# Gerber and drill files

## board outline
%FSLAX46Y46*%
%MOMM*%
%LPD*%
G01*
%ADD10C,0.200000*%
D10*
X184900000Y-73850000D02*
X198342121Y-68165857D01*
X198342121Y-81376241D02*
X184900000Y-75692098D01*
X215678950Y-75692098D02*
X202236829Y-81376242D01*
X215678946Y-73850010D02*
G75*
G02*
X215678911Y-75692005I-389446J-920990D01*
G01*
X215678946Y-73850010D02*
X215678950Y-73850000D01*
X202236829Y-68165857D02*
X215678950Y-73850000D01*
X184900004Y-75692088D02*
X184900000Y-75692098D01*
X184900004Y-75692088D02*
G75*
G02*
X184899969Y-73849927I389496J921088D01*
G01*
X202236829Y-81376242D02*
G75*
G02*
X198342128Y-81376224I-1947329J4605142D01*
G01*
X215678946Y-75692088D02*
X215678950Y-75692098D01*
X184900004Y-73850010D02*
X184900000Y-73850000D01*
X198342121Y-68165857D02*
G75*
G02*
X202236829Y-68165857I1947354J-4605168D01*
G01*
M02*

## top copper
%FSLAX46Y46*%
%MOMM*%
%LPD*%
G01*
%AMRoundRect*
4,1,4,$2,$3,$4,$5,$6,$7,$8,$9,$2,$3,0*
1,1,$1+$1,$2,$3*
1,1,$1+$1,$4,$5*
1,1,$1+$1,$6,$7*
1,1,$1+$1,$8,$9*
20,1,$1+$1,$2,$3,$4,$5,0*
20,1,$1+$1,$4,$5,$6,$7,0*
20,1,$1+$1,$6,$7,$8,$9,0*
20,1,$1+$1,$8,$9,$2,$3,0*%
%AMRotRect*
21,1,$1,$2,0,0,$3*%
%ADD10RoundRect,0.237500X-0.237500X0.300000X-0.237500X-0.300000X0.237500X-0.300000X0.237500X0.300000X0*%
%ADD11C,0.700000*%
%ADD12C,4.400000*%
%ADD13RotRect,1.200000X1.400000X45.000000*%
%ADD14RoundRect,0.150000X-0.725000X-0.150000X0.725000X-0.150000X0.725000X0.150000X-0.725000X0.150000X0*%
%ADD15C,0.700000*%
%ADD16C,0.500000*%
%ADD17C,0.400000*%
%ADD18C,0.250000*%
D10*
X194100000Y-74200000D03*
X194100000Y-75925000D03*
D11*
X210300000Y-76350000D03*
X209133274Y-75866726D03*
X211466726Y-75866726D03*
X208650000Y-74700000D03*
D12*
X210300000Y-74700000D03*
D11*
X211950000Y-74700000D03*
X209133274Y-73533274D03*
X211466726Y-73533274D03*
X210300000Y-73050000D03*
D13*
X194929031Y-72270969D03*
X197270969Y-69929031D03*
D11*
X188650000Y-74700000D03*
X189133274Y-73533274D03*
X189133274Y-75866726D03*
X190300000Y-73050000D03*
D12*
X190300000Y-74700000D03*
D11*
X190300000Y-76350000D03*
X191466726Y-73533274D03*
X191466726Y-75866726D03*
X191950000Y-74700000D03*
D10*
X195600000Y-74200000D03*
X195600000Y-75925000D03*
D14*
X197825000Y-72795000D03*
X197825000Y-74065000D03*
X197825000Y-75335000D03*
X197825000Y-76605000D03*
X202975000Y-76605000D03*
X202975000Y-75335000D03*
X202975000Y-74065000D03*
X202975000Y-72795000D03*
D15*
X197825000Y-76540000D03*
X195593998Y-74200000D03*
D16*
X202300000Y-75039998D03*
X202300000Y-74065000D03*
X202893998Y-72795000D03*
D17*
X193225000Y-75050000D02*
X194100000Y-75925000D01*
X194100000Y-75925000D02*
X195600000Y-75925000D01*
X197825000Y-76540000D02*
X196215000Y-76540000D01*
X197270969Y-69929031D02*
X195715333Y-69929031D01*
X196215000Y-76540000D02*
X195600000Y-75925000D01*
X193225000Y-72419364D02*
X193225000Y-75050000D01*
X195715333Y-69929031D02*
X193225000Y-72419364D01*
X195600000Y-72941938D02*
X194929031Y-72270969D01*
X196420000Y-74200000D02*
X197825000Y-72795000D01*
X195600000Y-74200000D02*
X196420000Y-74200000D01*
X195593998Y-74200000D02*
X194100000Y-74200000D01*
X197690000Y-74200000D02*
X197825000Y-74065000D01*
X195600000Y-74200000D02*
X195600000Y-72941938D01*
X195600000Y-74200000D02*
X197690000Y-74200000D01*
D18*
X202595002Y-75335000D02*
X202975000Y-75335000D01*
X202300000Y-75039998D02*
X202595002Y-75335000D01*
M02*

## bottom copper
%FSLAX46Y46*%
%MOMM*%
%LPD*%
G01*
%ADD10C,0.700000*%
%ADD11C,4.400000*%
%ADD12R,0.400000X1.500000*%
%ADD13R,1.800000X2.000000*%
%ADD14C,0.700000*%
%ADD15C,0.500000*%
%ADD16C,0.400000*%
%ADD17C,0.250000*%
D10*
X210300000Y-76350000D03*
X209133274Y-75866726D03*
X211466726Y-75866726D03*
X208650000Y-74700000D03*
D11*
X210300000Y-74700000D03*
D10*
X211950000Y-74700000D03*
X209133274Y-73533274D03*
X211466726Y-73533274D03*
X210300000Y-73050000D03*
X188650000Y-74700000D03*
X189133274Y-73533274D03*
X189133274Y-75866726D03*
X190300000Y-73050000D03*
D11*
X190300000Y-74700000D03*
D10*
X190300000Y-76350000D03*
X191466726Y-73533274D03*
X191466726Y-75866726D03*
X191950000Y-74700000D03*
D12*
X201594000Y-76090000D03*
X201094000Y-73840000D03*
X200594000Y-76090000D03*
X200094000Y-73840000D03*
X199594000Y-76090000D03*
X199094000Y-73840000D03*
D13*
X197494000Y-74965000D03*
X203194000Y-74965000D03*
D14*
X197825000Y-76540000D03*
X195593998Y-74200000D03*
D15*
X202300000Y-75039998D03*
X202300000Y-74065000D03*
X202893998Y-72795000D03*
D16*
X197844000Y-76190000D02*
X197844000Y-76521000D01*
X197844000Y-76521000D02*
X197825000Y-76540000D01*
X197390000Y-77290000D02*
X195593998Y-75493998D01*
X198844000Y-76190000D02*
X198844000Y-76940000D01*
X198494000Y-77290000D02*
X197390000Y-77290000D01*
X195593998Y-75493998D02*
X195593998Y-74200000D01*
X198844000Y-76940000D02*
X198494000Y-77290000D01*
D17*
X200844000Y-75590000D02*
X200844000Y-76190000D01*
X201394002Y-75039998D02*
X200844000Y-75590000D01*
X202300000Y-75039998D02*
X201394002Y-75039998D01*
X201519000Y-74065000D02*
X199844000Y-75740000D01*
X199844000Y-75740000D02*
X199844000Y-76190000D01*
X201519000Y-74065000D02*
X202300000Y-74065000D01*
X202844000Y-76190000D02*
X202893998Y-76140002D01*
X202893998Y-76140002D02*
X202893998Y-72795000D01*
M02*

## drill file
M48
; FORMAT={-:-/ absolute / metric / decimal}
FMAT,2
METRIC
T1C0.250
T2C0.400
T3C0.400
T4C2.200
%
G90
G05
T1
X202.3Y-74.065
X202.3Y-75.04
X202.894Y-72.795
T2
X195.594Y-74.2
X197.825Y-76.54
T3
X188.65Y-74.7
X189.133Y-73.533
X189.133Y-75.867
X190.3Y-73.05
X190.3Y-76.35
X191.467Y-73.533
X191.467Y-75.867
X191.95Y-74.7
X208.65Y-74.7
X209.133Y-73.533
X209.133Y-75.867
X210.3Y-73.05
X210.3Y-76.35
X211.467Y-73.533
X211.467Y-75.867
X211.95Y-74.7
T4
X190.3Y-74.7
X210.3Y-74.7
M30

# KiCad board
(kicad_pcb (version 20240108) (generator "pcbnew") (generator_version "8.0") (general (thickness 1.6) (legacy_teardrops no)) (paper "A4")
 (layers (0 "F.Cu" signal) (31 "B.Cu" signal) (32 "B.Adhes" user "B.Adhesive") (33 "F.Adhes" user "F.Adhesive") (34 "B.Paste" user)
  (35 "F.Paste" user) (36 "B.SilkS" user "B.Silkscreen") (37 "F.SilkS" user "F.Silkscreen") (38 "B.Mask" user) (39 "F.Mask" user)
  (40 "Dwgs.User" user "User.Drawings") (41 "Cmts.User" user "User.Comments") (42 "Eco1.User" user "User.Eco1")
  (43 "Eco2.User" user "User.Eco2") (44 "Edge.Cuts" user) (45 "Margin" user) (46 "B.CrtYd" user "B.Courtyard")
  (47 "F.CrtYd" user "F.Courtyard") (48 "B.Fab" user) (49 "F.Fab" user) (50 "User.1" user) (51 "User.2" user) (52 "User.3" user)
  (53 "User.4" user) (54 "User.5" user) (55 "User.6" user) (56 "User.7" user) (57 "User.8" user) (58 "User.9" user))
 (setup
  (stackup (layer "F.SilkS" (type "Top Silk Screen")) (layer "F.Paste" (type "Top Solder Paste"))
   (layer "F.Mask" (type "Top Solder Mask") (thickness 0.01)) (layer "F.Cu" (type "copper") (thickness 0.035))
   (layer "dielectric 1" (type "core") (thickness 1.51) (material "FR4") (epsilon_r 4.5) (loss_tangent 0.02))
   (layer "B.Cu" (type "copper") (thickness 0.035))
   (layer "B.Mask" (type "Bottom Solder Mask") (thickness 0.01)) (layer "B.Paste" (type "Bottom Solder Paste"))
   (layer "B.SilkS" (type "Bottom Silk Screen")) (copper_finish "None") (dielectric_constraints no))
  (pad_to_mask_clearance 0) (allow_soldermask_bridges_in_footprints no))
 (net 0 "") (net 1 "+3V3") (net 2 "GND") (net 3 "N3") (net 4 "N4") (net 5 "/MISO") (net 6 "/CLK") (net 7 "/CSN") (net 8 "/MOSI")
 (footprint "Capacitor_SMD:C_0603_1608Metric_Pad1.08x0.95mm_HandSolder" (layer "F.Cu") (at 194.1 75.0625 -90)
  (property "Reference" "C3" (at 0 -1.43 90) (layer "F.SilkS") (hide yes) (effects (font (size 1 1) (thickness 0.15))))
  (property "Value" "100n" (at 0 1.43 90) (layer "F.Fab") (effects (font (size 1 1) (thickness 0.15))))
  (pad "1" smd roundrect (at -0.8625 0 270) (size 1.075 0.95) (layers "F.Cu" "F.Paste" "F.Mask") (roundrect_rratio 0.25) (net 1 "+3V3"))
  (pad "2" smd roundrect (at 0.8625 0 270) (size 1.075 0.95) (layers "F.Cu" "F.Paste" "F.Mask") (roundrect_rratio 0.25) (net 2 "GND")))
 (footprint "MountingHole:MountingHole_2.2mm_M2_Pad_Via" (layer "F.Cu") (at 210.3 74.7 90)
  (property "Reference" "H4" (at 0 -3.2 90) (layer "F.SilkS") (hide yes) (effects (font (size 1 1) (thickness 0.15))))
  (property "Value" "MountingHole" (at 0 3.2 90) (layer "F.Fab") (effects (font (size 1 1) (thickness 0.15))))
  (pad "1" thru_hole circle (at -1.65 0 90) (size 0.7 0.7) (drill 0.4) (layers "*.Cu" "*.Mask") (remove_unused_layers no) (zone_connect 2))
  (pad "1" thru_hole circle (at -1.166726 -1.166726 90) (size 0.7 0.7) (drill 0.4) (layers "*.Cu" "*.Mask") (remove_unused_layers no)
   (zone_connect 2))
  (pad "1" thru_hole circle (at -1.166726 1.166726 90) (size 0.7 0.7) (drill 0.4) (layers "*.Cu" "*.Mask") (remove_unused_layers no)
   (zone_connect 2))
  (pad "1" thru_hole circle (at 0 -1.65 90) (size 0.7 0.7) (drill 0.4) (layers "*.Cu" "*.Mask") (remove_unused_layers no) (zone_connect 2))
  (pad "1" thru_hole circle (at 0 0 90) (size 4.4 4.4) (drill 2.2) (layers "*.Cu" "*.Mask") (remove_unused_layers no))
  (pad "1" thru_hole circle (at 0 1.65 90) (size 0.7 0.7) (drill 0.4) (layers "*.Cu" "*.Mask") (remove_unused_layers no) (zone_connect 2))
  (pad "1" thru_hole circle (at 1.166726 -1.166726 90) (size 0.7 0.7) (drill 0.4) (layers "*.Cu" "*.Mask") (remove_unused_layers no)
   (zone_connect 2))
  (pad "1" thru_hole circle (at 1.166726 1.166726 90) (size 0.7 0.7) (drill 0.4) (layers "*.Cu" "*.Mask") (remove_unused_layers no)
   (zone_connect 2))
  (pad "1" thru_hole circle (at 1.65 0 90) (size 0.7 0.7) (drill 0.4) (layers "*.Cu" "*.Mask") (remove_unused_layers no) (zone_connect 2)))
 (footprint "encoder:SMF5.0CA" (layer "F.Cu") (at 196.1 71.1 45)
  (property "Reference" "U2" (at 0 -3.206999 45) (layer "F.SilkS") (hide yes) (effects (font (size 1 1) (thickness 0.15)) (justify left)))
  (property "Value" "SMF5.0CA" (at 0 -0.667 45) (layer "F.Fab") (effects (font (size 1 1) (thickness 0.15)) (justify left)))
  (pad "1" smd rect (at -1.656 0 45) (size 1.2 1.4) (layers "F.Cu" "F.Paste" "F.Mask") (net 1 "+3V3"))
  (pad "2" smd rect (at 1.656 0 45) (size 1.2 1.4) (layers "F.Cu" "F.Paste" "F.Mask") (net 2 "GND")))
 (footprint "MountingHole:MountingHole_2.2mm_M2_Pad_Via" (layer "F.Cu") (at 190.3 74.7)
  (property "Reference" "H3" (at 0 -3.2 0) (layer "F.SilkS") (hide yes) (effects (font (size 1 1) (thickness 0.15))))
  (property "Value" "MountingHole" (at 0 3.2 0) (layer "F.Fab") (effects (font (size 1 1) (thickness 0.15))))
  (pad "1" thru_hole circle (at -1.65 0) (size 0.7 0.7) (drill 0.4) (layers "*.Cu" "*.Mask") (remove_unused_layers no) (zone_connect 2))
  (pad "1" thru_hole circle (at -1.166726 -1.166726) (size 0.7 0.7) (drill 0.4) (layers "*.Cu" "*.Mask") (remove_unused_layers no)
   (zone_connect 2))
  (pad "1" thru_hole circle (at -1.166726 1.166726) (size 0.7 0.7) (drill 0.4) (layers "*.Cu" "*.Mask") (remove_unused_layers no)
   (zone_connect 2))
  (pad "1" thru_hole circle (at 0 -1.65) (size 0.7 0.7) (drill 0.4) (layers "*.Cu" "*.Mask") (remove_unused_layers no) (zone_connect 2))
  (pad "1" thru_hole circle (at 0 0) (size 4.4 4.4) (drill 2.2) (layers "*.Cu" "*.Mask") (remove_unused_layers no))
  (pad "1" thru_hole circle (at 0 1.65) (size 0.7 0.7) (drill 0.4) (layers "*.Cu" "*.Mask") (remove_unused_layers no) (zone_connect 2))
  (pad "1" thru_hole circle (at 1.166726 -1.166726) (size 0.7 0.7) (drill 0.4) (layers "*.Cu" "*.Mask") (remove_unused_layers no)
   (zone_connect 2))
  (pad "1" thru_hole circle (at 1.166726 1.166726) (size 0.7 0.7) (drill 0.4) (layers "*.Cu" "*.Mask") (remove_unused_layers no)
   (zone_connect 2))
  (pad "1" thru_hole circle (at 1.65 0) (size 0.7 0.7) (drill 0.4) (layers "*.Cu" "*.Mask") (remove_unused_layers no) (zone_connect 2)))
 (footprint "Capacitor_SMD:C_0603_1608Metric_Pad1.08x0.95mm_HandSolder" (layer "F.Cu") (at 195.6 75.0625 -90)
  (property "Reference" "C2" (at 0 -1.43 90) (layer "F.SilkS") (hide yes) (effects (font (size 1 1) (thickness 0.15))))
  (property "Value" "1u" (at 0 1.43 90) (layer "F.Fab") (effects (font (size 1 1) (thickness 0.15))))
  (pad "1" smd roundrect (at -0.8625 0 270) (size 1.075 0.95) (layers "F.Cu" "F.Paste" "F.Mask") (roundrect_rratio 0.25) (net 1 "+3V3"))
  (pad "2" smd roundrect (at 0.8625 0 270) (size 1.075 0.95) (layers "F.Cu" "F.Paste" "F.Mask") (roundrect_rratio 0.25) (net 2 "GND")))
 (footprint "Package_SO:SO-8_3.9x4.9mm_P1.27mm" (layer "F.Cu") (at 200.4 74.7)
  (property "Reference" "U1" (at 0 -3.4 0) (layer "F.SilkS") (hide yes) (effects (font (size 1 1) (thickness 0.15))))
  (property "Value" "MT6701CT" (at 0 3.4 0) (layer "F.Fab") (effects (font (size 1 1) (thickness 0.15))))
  (pad "1" smd roundrect (at -2.575 -1.905) (size 1.75 0.6) (layers "F.Cu" "F.Paste" "F.Mask") (roundrect_rratio 0.25) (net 1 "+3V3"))
  (pad "2" smd roundrect (at -2.575 -0.635) (size 1.75 0.6) (layers "F.Cu" "F.Paste" "F.Mask") (roundrect_rratio 0.25) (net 1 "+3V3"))
  (pad "3" smd roundrect (at -2.575 0.635) (size 1.75 0.6) (layers "F.Cu" "F.Paste" "F.Mask") (roundrect_rratio 0.25) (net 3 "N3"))
  (pad "4" smd roundrect (at -2.575 1.905) (size 1.75 0.6) (layers "F.Cu" "F.Paste" "F.Mask") (roundrect_rratio 0.25) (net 2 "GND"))
  (pad "5" smd roundrect (at 2.575 1.905) (size 1.75 0.6) (layers "F.Cu" "F.Paste" "F.Mask") (roundrect_rratio 0.25) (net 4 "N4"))
  (pad "6" smd roundrect (at 2.575 0.635) (size 1.75 0.6) (layers "F.Cu" "F.Paste" "F.Mask") (roundrect_rratio 0.25) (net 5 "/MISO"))
  (pad "7" smd roundrect (at 2.575 -0.635) (size 1.75 0.6) (layers "F.Cu" "F.Paste" "F.Mask") (roundrect_rratio 0.25) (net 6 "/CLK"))
  (pad "8" smd roundrect (at 2.575 -1.905) (size 1.75 0.6) (layers "F.Cu" "F.Paste" "F.Mask") (roundrect_rratio 0.25) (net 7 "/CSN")))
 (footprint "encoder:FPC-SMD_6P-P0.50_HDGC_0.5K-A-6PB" (layer "B.Cu") (at 200.344 74.965 180)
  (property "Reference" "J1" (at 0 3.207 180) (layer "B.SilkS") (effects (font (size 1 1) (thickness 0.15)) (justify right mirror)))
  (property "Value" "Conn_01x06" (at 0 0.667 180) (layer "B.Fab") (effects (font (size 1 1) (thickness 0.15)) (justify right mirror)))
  (pad "1" smd rect (at -1.25 -1.125) (size 0.4 1.5) (layers "B.Cu" "B.Paste" "B.Mask") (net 7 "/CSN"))
  (pad "2" smd rect (at -0.75 1.125) (size 0.4 1.5) (layers "B.Cu" "B.Paste" "B.Mask") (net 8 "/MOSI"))
  (pad "3" smd rect (at -0.25 -1.125) (size 0.4 1.5) (layers "B.Cu" "B.Paste" "B.Mask") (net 5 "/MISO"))
  (pad "4" smd rect (at 0.25 1.125) (size 0.4 1.5) (layers "B.Cu" "B.Paste" "B.Mask") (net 6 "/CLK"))
  (pad "5" smd rect (at 0.75 -1.125) (size 0.4 1.5) (layers "B.Cu" "B.Paste" "B.Mask") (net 1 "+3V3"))
  (pad "6" smd rect (at 1.25 1.125) (size 0.4 1.5) (layers "B.Cu" "B.Paste" "B.Mask") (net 2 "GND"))
  (pad "7" smd rect (at 2.85 0) (size 1.8 2) (layers "B.Cu" "B.Paste" "B.Mask"))
  (pad "8" smd rect (at -2.85 0 180) (size 1.8 2) (layers "B.Cu" "B.Paste" "B.Mask")))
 (gr_line (start 184.9 73.85) (end 198.342121 68.165857) (stroke (width 0.2) (type default)) (layer "Edge.Cuts"))
 (gr_line (start 198.342121 81.376241) (end 184.9 75.692098) (stroke (width 0.2) (type default)) (layer "Edge.Cuts"))
 (gr_line (start 215.67895 75.692098) (end 202.236829 81.376242) (stroke (width 0.2) (type default)) (layer "Edge.Cuts"))
 (gr_arc (start 215.678946 73.85001) (mid 216.289475 74.771049) (end 215.678946 75.692088) (stroke (width 0.2) (type default))
  (layer "Edge.Cuts"))
 (gr_line (start 215.678946 73.85001) (end 215.67895 73.85) (stroke (width 0.2) (type default)) (layer "Edge.Cuts"))
 (gr_line (start 202.236829 68.165857) (end 215.67895 73.85) (stroke (width 0.2) (type default)) (layer "Edge.Cuts"))
 (gr_line (start 184.900004 75.692088) (end 184.9 75.692098) (stroke (width 0.2) (type default)) (layer "Edge.Cuts"))
 (gr_arc (start 184.900004 75.692088) (mid 184.289475 74.771049) (end 184.900004 73.85001) (stroke (width 0.2) (type default))
  (layer "Edge.Cuts"))
 (gr_arc (start 202.236829 81.376242) (mid 200.289475 81.771049) (end 198.342121 81.376241) (stroke (width 0.2) (type default))
  (layer "Edge.Cuts"))
 (gr_line (start 215.678946 75.692088) (end 215.67895 75.692098) (stroke (width 0.2) (type default)) (layer "Edge.Cuts"))
 (gr_line (start 184.900004 73.85001) (end 184.9 73.85) (stroke (width 0.2) (type default)) (layer "Edge.Cuts"))
 (gr_arc (start 198.342121 68.165857) (mid 200.289475 67.771049) (end 202.236829 68.165857) (stroke (width 0.2) (type default))
  (layer "Edge.Cuts"))
 (segment (start 193.225 75.05) (end 194.1 75.925) (width 0.4) (layer "F.Cu") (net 2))
 (segment (start 194.1 75.925) (end 195.6 75.925) (width 0.4) (layer "F.Cu") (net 2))
 (segment (start 197.825 76.54) (end 196.215 76.54) (width 0.4) (layer "F.Cu") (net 2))
 (segment (start 197.270969 69.929031) (end 195.715333 69.929031) (width 0.4) (layer "F.Cu") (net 2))
 (segment (start 196.215 76.54) (end 195.6 75.925) (width 0.4) (layer "F.Cu") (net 2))
 (segment (start 193.225 72.419364) (end 193.225 75.05) (width 0.4) (layer "F.Cu") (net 2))
 (segment (start 195.715333 69.929031) (end 193.225 72.419364) (width 0.4) (layer "F.Cu") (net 2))
 (via blind (at 197.825 76.54) (size 0.7) (drill 0.4) (layers "F.Cu" "B.Cu") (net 2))
 (segment (start 197.844 76.19) (end 197.844 76.521) (width 0.4) (layer "B.Cu") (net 2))
 (segment (start 197.844 76.521) (end 197.825 76.54) (width 0.4) (layer "B.Cu") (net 2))
 (segment (start 195.6 72.941938) (end 194.929031 72.270969) (width 0.4) (layer "F.Cu") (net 1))
 (segment (start 196.42 74.2) (end 197.825 72.795) (width 0.4) (layer "F.Cu") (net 1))
 (segment (start 195.6 74.2) (end 196.42 74.2) (width 0.4) (layer "F.Cu") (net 1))
 (segment (start 195.593998 74.2) (end 194.1 74.2) (width 0.4) (layer "F.Cu") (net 1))
 (segment (start 197.69 74.2) (end 197.825 74.065) (width 0.4) (layer "F.Cu") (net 1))
 (segment (start 195.6 74.2) (end 195.6 72.941938) (width 0.4) (layer "F.Cu") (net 1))
 (segment (start 195.6 74.2) (end 197.69 74.2) (width 0.4) (layer "F.Cu") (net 1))
 (via blind (at 195.593998 74.2) (size 0.7) (drill 0.4) (layers "F.Cu" "B.Cu") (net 1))
 (segment (start 197.39 77.29) (end 195.593998 75.493998) (width 0.4) (layer "B.Cu") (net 1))
 (segment (start 198.844 76.19) (end 198.844 76.94) (width 0.4) (layer "B.Cu") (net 1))
 (segment (start 198.494 77.29) (end 197.39 77.29) (width 0.4) (layer "B.Cu") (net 1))
 (segment (start 195.593998 75.493998) (end 195.593998 74.2) (width 0.4) (layer "B.Cu") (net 1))
 (segment (start 198.844 76.94) (end 198.494 77.29) (width 0.4) (layer "B.Cu") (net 1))
 (segment (start 202.595002 75.335) (end 202.975 75.335) (width 0.25) (layer "F.Cu") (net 5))
 (segment (start 202.3 75.039998) (end 202.595002 75.335) (width 0.25) (layer "F.Cu") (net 5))
 (via blind (at 202.3 75.039998) (size 0.5) (drill 0.25) (layers "F.Cu" "B.Cu") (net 5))
 (segment (start 200.844 75.59) (end 200.844 76.19) (width 0.25) (layer "B.Cu") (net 5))
 (segment (start 201.394002 75.039998) (end 200.844 75.59) (width 0.25) (layer "B.Cu") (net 5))
 (segment (start 202.3 75.039998) (end 201.394002 75.039998) (width 0.25) (layer "B.Cu") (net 5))
 (via blind (at 202.3 74.065) (size 0.5) (drill 0.25) (layers "F.Cu" "B.Cu") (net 6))
 (segment (start 201.519 74.065) (end 199.844 75.74) (width 0.25) (layer "B.Cu") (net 6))
 (segment (start 199.844 75.74) (end 199.844 76.19) (width 0.25) (layer "B.Cu") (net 6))
 (segment (start 201.519 74.065) (end 202.3 74.065) (width 0.25) (layer "B.Cu") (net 6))
 (via blind (at 202.893998 72.795) (size 0.5) (drill 0.25) (layers "F.Cu" "B.Cu") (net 7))
 (segment (start 202.844 76.19) (end 202.893998 76.140002) (width 0.25) (layer "B.Cu") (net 7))
 (segment (start 202.893998 76.140002) (end 202.893998 72.795) (width 0.25) (layer "B.Cu") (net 7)))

